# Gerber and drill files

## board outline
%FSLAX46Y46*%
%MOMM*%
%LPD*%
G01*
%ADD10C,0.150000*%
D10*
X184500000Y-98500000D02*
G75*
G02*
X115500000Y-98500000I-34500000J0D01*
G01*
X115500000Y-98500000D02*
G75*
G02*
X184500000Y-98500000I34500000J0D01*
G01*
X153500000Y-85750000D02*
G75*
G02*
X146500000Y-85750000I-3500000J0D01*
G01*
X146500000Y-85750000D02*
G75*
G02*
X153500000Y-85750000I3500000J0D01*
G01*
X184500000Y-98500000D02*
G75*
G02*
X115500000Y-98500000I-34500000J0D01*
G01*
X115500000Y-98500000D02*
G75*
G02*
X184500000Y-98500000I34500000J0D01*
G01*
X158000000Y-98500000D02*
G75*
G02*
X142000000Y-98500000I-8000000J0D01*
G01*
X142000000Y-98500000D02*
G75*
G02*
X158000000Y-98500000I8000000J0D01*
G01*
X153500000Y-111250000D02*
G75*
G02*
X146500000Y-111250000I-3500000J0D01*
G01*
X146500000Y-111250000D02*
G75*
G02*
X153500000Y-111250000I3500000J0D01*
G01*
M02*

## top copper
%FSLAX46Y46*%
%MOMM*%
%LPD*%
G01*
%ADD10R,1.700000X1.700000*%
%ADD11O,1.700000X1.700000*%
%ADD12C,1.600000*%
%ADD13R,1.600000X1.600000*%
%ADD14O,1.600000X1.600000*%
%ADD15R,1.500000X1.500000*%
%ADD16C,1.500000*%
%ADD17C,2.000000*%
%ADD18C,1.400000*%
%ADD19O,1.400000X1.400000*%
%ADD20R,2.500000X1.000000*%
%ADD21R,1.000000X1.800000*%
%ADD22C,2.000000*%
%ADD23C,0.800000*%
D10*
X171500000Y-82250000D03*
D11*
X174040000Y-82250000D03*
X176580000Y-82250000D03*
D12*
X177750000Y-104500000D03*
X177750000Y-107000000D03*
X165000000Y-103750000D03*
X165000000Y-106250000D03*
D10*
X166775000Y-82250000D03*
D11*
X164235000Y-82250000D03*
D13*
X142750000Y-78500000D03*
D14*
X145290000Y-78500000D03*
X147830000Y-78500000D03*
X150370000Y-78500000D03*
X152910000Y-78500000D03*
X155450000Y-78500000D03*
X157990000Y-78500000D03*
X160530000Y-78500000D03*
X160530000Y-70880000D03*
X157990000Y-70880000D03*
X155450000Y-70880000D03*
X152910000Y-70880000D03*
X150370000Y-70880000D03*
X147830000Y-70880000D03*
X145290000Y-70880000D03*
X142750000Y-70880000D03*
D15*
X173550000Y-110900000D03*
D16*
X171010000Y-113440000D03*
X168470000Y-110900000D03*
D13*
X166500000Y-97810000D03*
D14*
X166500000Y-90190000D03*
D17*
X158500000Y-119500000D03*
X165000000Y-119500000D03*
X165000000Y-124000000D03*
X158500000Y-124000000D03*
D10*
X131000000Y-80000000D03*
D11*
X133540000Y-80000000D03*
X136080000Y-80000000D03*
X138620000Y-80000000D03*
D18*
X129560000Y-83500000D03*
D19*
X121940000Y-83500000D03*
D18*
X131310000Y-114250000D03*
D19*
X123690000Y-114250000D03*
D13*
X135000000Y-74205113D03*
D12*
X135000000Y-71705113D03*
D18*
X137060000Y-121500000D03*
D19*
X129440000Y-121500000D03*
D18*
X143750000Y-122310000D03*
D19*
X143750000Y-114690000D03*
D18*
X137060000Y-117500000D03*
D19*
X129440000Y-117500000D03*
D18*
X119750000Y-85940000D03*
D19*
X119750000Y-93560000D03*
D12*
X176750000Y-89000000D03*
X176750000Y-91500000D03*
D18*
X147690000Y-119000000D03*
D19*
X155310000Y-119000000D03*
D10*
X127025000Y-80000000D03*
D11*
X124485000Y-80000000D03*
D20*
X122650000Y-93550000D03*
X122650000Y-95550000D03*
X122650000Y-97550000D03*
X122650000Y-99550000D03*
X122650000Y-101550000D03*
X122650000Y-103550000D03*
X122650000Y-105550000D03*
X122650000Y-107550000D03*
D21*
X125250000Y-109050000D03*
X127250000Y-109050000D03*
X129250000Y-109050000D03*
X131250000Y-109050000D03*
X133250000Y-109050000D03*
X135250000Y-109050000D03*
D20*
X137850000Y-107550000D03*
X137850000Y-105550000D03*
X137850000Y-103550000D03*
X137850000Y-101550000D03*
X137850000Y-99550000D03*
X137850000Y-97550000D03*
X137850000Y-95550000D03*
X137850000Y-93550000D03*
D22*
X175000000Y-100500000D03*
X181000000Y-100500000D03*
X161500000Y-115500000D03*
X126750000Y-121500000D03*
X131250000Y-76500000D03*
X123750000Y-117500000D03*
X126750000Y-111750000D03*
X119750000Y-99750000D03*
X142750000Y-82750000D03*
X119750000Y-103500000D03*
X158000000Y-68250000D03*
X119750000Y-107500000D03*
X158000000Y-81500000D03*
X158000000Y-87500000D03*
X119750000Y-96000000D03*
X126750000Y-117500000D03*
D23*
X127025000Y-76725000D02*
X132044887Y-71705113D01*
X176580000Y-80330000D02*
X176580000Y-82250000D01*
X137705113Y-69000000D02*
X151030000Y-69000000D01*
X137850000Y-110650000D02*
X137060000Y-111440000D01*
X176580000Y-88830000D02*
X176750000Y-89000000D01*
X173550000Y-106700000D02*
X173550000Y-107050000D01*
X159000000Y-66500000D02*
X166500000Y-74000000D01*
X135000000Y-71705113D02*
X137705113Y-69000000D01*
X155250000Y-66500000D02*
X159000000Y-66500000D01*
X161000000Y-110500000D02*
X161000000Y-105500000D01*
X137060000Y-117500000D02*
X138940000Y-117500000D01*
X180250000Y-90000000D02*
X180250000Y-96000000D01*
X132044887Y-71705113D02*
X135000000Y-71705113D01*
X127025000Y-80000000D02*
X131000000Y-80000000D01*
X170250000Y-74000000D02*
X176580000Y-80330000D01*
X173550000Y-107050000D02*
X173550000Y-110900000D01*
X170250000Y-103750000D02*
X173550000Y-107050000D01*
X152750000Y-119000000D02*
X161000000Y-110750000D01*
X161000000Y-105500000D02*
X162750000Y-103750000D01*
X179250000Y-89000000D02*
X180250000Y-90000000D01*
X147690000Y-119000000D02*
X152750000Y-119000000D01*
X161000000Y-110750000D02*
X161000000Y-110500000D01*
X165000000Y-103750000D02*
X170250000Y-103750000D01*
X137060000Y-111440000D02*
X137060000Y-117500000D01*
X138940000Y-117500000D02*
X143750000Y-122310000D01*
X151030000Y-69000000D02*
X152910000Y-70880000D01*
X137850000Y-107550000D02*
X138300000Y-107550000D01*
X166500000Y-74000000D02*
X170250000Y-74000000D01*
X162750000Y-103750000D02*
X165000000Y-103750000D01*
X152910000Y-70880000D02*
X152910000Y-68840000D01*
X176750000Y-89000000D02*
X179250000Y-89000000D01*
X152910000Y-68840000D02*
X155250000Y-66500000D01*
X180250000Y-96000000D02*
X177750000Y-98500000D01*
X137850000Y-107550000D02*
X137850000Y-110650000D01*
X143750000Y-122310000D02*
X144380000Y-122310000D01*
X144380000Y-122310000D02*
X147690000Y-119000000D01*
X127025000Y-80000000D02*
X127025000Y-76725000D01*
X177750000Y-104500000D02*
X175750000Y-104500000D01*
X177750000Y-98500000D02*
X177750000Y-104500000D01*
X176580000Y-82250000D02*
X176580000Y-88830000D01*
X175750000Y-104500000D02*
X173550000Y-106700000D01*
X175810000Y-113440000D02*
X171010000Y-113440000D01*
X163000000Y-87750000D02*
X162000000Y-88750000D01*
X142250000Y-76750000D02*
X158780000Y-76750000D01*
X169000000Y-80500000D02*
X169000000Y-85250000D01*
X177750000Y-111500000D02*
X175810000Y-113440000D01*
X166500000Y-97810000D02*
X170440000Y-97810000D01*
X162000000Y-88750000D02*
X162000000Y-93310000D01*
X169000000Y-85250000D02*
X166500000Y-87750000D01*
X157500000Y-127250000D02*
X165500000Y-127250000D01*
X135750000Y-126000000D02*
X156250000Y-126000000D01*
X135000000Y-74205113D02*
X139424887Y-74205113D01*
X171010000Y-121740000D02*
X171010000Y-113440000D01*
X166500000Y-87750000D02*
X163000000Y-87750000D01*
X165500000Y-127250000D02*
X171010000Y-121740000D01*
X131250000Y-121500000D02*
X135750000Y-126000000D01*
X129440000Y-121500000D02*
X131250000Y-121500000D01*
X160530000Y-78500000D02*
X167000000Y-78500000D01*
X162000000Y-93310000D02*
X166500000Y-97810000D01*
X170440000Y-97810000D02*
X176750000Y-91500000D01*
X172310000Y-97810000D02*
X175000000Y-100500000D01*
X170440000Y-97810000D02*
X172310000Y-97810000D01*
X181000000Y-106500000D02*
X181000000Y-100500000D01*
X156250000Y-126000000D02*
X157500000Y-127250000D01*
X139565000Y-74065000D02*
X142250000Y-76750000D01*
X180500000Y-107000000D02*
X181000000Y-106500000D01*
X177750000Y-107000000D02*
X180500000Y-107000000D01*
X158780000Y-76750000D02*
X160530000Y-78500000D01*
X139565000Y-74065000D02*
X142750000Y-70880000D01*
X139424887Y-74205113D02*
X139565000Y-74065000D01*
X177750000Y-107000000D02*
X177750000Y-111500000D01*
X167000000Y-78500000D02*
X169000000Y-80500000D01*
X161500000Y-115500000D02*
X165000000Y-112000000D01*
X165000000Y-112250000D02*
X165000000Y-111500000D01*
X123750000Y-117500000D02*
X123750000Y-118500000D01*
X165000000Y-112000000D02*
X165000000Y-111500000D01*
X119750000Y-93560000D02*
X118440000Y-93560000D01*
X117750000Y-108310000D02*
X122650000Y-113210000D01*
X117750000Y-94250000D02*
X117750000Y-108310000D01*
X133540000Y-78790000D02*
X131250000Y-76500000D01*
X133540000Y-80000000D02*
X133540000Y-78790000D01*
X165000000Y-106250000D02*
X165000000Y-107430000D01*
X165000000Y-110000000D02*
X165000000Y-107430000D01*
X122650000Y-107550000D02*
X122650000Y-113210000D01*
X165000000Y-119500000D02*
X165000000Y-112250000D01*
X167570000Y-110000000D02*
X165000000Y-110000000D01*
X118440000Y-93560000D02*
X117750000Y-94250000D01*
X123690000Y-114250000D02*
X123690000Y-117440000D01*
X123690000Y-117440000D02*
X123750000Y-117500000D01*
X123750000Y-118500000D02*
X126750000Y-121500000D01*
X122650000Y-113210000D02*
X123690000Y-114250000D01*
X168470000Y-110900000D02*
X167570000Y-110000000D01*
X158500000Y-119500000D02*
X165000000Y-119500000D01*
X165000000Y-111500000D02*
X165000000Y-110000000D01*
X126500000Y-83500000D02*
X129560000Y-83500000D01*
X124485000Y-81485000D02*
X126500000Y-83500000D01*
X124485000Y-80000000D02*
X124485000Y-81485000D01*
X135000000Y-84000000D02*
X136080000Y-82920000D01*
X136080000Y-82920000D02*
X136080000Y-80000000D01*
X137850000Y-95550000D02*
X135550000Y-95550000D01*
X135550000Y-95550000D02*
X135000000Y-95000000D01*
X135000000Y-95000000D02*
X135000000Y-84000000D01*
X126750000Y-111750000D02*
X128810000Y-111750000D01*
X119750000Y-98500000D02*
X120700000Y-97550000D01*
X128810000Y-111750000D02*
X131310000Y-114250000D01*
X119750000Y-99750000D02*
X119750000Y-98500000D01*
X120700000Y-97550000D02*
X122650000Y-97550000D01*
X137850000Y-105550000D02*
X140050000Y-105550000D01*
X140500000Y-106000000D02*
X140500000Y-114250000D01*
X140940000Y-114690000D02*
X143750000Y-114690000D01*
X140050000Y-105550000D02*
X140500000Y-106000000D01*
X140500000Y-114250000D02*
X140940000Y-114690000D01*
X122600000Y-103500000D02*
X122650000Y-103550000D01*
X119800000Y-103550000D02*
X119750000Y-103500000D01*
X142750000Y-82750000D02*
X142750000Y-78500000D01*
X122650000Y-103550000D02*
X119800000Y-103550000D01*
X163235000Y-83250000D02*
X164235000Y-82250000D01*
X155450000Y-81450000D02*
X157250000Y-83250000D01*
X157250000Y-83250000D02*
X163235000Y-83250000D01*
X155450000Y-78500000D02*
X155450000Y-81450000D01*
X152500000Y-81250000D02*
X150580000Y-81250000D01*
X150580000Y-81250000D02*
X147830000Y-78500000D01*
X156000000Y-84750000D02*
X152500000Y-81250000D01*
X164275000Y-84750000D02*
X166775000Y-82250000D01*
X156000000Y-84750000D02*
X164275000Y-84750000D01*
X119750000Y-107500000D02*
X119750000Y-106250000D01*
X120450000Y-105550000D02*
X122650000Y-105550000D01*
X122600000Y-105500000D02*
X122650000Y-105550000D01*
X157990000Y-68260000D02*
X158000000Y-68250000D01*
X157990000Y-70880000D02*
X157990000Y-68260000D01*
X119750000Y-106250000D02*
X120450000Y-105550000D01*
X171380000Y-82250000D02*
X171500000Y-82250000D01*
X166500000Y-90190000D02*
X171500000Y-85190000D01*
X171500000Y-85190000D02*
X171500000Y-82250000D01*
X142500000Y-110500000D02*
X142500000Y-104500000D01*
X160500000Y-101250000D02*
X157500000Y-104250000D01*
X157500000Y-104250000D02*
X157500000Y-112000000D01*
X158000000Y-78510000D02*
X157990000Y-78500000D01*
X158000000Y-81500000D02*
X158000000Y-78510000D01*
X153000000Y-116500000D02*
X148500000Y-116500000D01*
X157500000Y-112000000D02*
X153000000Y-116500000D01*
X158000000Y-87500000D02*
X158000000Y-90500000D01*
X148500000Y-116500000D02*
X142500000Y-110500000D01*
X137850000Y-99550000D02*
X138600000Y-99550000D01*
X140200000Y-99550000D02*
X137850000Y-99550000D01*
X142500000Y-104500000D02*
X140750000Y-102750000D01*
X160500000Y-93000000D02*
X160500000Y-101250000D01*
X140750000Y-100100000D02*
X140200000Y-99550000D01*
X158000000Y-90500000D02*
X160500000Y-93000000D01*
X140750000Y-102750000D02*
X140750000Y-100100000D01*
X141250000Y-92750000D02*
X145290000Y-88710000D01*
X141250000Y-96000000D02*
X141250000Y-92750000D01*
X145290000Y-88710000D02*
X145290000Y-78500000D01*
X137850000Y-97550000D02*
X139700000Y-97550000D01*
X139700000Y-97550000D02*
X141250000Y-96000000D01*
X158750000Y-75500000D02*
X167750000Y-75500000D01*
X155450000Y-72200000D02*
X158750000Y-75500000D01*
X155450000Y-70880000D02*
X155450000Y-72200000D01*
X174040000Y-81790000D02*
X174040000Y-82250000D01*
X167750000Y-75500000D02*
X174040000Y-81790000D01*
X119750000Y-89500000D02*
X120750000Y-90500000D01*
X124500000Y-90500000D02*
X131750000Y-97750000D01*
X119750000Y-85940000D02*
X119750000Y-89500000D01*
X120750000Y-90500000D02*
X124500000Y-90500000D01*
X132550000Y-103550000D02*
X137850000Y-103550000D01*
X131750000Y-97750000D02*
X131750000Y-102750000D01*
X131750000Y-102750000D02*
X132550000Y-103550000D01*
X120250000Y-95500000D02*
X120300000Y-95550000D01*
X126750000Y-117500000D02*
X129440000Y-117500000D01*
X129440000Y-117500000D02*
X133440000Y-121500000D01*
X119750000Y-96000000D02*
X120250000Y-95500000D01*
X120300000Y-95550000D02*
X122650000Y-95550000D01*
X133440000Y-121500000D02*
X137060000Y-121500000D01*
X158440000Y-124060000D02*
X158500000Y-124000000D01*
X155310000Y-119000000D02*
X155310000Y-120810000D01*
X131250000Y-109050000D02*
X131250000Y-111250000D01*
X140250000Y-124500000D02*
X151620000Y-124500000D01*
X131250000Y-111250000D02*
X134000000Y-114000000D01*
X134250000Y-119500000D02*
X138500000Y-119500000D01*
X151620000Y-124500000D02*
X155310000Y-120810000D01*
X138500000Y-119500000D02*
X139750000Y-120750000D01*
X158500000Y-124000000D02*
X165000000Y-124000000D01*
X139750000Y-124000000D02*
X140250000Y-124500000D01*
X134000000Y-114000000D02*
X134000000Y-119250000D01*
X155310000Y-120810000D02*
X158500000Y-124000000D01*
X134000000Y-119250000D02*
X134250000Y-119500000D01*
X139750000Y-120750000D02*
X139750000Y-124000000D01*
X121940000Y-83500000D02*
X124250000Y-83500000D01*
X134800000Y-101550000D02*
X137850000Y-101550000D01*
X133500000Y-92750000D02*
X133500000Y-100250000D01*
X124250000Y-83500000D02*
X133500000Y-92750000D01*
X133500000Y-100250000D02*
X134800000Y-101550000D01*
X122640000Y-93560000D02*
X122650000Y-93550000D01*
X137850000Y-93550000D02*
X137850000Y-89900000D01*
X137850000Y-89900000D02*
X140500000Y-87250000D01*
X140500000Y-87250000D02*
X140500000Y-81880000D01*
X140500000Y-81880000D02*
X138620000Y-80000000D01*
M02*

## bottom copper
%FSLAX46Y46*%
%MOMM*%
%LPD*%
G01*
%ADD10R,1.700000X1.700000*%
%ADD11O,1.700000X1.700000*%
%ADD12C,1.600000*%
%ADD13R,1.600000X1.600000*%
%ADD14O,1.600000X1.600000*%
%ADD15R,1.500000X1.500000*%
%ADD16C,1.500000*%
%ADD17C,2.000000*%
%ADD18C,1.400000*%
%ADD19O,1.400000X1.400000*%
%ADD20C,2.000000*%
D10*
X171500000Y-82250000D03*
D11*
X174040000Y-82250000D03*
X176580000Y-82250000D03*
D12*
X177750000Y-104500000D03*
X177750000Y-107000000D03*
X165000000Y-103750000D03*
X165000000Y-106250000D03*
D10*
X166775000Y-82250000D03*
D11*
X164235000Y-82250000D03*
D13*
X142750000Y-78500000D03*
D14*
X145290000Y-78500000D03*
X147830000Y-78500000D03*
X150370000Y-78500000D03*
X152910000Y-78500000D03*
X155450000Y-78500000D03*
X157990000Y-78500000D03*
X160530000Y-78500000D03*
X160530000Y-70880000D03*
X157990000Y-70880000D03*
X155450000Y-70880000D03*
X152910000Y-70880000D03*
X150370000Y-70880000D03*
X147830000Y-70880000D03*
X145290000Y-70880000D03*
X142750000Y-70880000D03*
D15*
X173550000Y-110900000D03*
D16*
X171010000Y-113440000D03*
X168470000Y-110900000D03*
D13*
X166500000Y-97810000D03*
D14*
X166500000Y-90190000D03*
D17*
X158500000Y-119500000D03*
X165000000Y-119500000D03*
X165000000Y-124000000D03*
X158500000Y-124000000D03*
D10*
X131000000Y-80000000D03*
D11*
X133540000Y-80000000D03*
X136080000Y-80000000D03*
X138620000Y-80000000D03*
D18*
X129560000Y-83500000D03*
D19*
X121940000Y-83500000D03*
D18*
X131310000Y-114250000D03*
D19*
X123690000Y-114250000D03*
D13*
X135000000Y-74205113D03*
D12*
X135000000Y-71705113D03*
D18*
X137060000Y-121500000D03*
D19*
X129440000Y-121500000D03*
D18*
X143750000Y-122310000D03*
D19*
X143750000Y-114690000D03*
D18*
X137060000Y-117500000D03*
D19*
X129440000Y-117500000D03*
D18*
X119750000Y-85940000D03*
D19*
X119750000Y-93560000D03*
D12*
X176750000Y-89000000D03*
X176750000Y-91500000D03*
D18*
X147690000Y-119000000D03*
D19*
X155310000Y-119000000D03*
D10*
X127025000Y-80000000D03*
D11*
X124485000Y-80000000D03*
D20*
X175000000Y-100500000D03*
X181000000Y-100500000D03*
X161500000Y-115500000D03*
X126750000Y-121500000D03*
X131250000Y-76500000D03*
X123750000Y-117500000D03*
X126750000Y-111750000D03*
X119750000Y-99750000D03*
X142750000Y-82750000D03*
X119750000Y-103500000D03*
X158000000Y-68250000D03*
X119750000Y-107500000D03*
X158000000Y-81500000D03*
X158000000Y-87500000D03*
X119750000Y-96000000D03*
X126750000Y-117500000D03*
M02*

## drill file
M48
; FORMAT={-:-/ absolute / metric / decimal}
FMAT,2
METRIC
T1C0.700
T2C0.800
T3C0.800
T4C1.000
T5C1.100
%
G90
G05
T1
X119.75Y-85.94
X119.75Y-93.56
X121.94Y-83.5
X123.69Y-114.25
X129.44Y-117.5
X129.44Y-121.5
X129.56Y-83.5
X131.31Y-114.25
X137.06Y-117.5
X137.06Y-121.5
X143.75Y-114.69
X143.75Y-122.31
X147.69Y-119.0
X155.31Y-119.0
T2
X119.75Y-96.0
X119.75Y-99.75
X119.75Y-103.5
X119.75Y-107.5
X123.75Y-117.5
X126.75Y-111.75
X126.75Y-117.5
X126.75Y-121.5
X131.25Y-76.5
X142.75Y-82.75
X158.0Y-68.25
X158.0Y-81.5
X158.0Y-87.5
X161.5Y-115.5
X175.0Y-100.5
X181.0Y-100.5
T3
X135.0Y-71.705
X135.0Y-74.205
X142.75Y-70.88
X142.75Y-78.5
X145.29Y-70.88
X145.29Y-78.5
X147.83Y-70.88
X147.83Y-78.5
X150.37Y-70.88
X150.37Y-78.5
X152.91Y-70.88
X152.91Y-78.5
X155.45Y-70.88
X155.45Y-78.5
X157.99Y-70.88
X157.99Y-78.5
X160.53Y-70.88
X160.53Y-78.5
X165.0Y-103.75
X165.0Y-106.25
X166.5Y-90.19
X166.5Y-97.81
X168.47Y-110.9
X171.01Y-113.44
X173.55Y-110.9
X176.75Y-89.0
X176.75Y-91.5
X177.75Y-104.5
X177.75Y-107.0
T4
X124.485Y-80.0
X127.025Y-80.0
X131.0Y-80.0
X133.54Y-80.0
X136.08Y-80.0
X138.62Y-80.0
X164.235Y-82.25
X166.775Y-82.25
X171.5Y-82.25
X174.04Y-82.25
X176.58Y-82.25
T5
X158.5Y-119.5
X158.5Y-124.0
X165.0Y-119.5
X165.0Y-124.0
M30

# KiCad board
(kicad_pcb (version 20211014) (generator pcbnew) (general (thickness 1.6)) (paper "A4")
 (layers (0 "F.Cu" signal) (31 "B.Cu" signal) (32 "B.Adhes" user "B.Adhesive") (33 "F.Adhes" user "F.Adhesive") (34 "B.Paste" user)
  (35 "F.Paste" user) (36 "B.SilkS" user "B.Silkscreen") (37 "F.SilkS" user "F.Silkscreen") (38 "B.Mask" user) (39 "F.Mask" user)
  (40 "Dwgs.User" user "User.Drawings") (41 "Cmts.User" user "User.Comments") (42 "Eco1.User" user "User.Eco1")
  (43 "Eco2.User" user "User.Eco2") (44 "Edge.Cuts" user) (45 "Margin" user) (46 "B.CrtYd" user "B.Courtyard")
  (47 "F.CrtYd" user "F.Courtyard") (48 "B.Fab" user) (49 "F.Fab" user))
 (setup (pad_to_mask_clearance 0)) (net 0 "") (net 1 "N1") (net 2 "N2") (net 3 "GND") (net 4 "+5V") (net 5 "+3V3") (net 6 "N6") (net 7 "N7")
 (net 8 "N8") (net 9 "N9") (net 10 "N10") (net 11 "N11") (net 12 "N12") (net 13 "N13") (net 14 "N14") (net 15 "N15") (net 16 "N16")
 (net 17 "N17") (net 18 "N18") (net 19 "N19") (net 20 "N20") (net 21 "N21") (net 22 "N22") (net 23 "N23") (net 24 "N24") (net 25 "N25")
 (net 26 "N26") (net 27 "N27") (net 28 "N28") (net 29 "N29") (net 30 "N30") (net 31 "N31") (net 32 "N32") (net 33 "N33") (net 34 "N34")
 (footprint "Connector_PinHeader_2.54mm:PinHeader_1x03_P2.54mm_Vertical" (layer "F.Cu") (at 171.5 82.25 90)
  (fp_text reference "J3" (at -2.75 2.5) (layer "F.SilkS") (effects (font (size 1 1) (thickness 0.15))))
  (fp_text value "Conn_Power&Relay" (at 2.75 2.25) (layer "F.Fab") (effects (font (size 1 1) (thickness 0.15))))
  (pad "1" thru_hole rect locked (at 0 0 90) (size 1.7 1.7) (drill 1) (layers *.Cu *.Mask) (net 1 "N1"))
  (pad "2" thru_hole oval locked (at 0 2.54 90) (size 1.7 1.7) (drill 1) (layers *.Cu *.Mask) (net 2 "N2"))
  (pad "3" thru_hole oval locked (at 0 5.08 90) (size 1.7 1.7) (drill 1) (layers *.Cu *.Mask) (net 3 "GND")))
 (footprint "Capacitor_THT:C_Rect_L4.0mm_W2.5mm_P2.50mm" (layer "F.Cu") (at 177.75 104.5 -90)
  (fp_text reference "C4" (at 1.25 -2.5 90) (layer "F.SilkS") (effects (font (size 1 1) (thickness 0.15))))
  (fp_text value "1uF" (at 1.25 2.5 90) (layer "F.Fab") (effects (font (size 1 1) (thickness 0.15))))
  (pad "1" thru_hole circle locked (at 0 0 270) (size 1.6 1.6) (drill 0.8) (layers *.Cu *.Mask) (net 3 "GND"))
  (pad "2" thru_hole circle locked (at 2.5 0 270) (size 1.6 1.6) (drill 0.8) (layers *.Cu *.Mask) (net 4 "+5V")))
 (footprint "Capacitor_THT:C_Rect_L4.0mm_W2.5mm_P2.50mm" (layer "F.Cu") (at 165 103.75 -90)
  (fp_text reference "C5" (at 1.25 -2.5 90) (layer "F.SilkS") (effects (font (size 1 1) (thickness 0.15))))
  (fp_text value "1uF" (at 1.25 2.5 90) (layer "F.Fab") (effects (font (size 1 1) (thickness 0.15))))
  (pad "1" thru_hole circle locked (at 0 0 270) (size 1.6 1.6) (drill 0.8) (layers *.Cu *.Mask) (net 3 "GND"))
  (pad "2" thru_hole circle locked (at 2.5 0 270) (size 1.6 1.6) (drill 0.8) (layers *.Cu *.Mask) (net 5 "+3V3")))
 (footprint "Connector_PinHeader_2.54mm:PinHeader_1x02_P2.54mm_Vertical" (layer "F.Cu") (at 166.775 82.25 -90)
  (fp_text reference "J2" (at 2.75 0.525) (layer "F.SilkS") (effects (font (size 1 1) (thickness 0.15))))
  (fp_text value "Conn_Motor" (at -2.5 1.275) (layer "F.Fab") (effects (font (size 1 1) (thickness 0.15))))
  (pad "1" thru_hole rect locked (at 0 0 270) (size 1.7 1.7) (drill 1) (layers *.Cu *.Mask) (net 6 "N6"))
  (pad "2" thru_hole oval locked (at 0 2.54 270) (size 1.7 1.7) (drill 1) (layers *.Cu *.Mask) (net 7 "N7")))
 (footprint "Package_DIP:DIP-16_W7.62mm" (layer "F.Cu") (at 142.75 78.5 90)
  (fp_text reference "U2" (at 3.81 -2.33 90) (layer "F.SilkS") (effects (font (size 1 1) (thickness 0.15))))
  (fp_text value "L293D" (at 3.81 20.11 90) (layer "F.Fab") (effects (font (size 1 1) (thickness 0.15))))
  (pad "1" thru_hole rect locked (at 0 0 90) (size 1.6 1.6) (drill 0.8) (layers *.Cu *.Mask) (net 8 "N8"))
  (pad "2" thru_hole oval locked (at 0 2.54 90) (size 1.6 1.6) (drill 0.8) (layers *.Cu *.Mask) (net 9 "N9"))
  (pad "3" thru_hole oval locked (at 0 5.08 90) (size 1.6 1.6) (drill 0.8) (layers *.Cu *.Mask) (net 6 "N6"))
  (pad "4" thru_hole oval locked (at 0 7.62 90) (size 1.6 1.6) (drill 0.8) (layers *.Cu *.Mask) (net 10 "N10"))
  (pad "5" thru_hole oval locked (at 0 10.16 90) (size 1.6 1.6) (drill 0.8) (layers *.Cu *.Mask) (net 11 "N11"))
  (pad "6" thru_hole oval locked (at 0 12.7 90) (size 1.6 1.6) (drill 0.8) (layers *.Cu *.Mask) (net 7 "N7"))
  (pad "7" thru_hole oval locked (at 0 15.24 90) (size 1.6 1.6) (drill 0.8) (layers *.Cu *.Mask) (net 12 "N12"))
  (pad "8" thru_hole oval locked (at 0 17.78 90) (size 1.6 1.6) (drill 0.8) (layers *.Cu *.Mask) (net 4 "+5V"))
  (pad "9" thru_hole oval locked (at 7.62 17.78 90) (size 1.6 1.6) (drill 0.8) (layers *.Cu *.Mask) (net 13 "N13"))
  (pad "10" thru_hole oval locked (at 7.62 15.24 90) (size 1.6 1.6) (drill 0.8) (layers *.Cu *.Mask) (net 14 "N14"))
  (pad "11" thru_hole oval locked (at 7.62 12.7 90) (size 1.6 1.6) (drill 0.8) (layers *.Cu *.Mask) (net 2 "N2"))
  (pad "12" thru_hole oval locked (at 7.62 10.16 90) (size 1.6 1.6) (drill 0.8) (layers *.Cu *.Mask) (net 3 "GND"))
  (pad "13" thru_hole oval locked (at 7.62 7.62 90) (size 1.6 1.6) (drill 0.8) (layers *.Cu *.Mask) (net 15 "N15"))
  (pad "14" thru_hole oval locked (at 7.62 5.08 90) (size 1.6 1.6) (drill 0.8) (layers *.Cu *.Mask) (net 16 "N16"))
  (pad "15" thru_hole oval locked (at 7.62 2.54 90) (size 1.6 1.6) (drill 0.8) (layers *.Cu *.Mask) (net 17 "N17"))
  (pad "16" thru_hole oval locked (at 7.62 0 90) (size 1.6 1.6) (drill 0.8) (layers *.Cu *.Mask) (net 4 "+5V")))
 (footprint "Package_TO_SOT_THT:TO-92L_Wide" (layer "F.Cu") (at 173.55 110.9 180)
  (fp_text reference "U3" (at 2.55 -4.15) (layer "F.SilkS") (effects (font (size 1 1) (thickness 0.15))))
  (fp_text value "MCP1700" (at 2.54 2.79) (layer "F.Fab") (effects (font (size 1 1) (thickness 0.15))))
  (pad "1" thru_hole rect locked (at 0 0 180) (size 1.5 1.5) (drill 0.8) (layers *.Cu *.Mask) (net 3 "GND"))
  (pad "2" thru_hole circle locked (at 2.54 -2.54 180) (size 1.5 1.5) (drill 0.8) (layers *.Cu *.Mask) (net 4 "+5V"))
  (pad "3" thru_hole circle locked (at 5.08 0 180) (size 1.5 1.5) (drill 0.8) (layers *.Cu *.Mask) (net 5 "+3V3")))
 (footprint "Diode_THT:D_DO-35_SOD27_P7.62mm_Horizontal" (layer "F.Cu") (at 166.5 97.81 90)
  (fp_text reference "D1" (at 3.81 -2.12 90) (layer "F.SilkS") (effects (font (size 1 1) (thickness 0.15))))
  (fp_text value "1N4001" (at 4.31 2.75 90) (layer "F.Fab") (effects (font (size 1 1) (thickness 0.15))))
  (pad "1" thru_hole rect locked (at 0 0 90) (size 1.6 1.6) (drill 0.8) (layers *.Cu *.Mask) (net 4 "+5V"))
  (pad "2" thru_hole oval locked (at 7.62 0 90) (size 1.6 1.6) (drill 0.8) (layers *.Cu *.Mask) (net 1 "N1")))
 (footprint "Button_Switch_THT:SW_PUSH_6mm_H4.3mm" (layer "F.Cu") (at 158.5 119.5)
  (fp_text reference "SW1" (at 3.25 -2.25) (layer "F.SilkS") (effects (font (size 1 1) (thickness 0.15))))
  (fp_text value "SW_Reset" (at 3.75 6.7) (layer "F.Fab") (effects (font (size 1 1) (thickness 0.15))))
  (pad "1" thru_hole circle locked (at 0 0 90) (size 2 2) (drill 1.1) (layers *.Cu *.Mask) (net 5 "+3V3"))
  (pad "1" thru_hole circle locked (at 6.5 0 90) (size 2 2) (drill 1.1) (layers *.Cu *.Mask) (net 5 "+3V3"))
  (pad "2" thru_hole circle locked (at 6.5 4.5 90) (size 2 2) (drill 1.1) (layers *.Cu *.Mask) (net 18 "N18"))
  (pad "2" thru_hole circle locked (at 0 4.5 90) (size 2 2) (drill 1.1) (layers *.Cu *.Mask) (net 18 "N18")))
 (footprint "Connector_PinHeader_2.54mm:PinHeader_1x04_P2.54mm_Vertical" (layer "F.Cu") (at 131 80 90)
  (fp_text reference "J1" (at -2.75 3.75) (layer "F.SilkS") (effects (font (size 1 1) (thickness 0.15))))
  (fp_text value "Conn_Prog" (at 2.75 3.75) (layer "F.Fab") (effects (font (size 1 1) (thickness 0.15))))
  (pad "1" thru_hole rect locked (at 0 0 90) (size 1.7 1.7) (drill 1) (layers *.Cu *.Mask) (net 3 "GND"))
  (pad "2" thru_hole oval locked (at 0 2.54 90) (size 1.7 1.7) (drill 1) (layers *.Cu *.Mask) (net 5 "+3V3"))
  (pad "3" thru_hole oval locked (at 0 5.08 90) (size 1.7 1.7) (drill 1) (layers *.Cu *.Mask) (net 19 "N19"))
  (pad "4" thru_hole oval locked (at 0 7.62 90) (size 1.7 1.7) (drill 1) (layers *.Cu *.Mask) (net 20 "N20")))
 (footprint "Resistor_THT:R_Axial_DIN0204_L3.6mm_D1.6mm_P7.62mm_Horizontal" (layer "F.Cu") (at 129.56 83.5 180)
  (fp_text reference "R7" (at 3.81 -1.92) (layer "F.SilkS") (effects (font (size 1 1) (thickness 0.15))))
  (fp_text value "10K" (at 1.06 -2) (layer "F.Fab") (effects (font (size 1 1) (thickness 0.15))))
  (pad "1" thru_hole circle locked (at 0 0 180) (size 1.4 1.4) (drill 0.7) (layers *.Cu *.Mask) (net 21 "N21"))
  (pad "2" thru_hole oval locked (at 7.62 0 180) (size 1.4 1.4) (drill 0.7) (layers *.Cu *.Mask) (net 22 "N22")))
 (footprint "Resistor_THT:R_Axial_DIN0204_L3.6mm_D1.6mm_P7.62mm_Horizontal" (layer "F.Cu") (at 131.31 114.25 180)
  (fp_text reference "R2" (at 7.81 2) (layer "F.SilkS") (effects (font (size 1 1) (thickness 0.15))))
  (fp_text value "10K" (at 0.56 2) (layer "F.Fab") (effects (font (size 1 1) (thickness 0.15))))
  (pad "1" thru_hole circle locked (at 0 0 180) (size 1.4 1.4) (drill 0.7) (layers *.Cu *.Mask) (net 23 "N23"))
  (pad "2" thru_hole oval locked (at 7.62 0 180) (size 1.4 1.4) (drill 0.7) (layers *.Cu *.Mask) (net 5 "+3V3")))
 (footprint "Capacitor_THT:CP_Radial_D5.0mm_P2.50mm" (layer "F.Cu") (at 135 74.205113 90)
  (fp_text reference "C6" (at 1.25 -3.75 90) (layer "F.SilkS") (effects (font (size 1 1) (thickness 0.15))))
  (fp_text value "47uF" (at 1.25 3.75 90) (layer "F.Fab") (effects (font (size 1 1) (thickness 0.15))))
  (pad "1" thru_hole rect locked (at 0 0 90) (size 1.6 1.6) (drill 0.8) (layers *.Cu *.Mask) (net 4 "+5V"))
  (pad "2" thru_hole circle locked (at 2.5 0 90) (size 1.6 1.6) (drill 0.8) (layers *.Cu *.Mask) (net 3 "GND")))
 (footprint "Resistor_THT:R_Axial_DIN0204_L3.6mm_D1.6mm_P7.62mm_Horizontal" (layer "F.Cu") (at 137.06 121.5 180)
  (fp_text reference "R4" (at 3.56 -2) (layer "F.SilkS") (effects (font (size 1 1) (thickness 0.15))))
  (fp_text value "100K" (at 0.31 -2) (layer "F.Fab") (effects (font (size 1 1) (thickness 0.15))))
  (pad "1" thru_hole circle locked (at 0 0 180) (size 1.4 1.4) (drill 0.7) (layers *.Cu *.Mask) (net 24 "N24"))
  (pad "2" thru_hole oval locked (at 7.62 0 180) (size 1.4 1.4) (drill 0.7) (layers *.Cu *.Mask) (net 4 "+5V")))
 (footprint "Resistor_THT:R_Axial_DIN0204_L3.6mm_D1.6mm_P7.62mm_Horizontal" (layer "F.Cu") (at 143.75 122.31 90)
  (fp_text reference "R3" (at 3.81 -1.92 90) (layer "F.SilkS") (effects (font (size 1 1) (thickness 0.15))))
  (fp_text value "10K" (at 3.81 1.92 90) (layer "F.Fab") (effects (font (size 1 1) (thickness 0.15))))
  (pad "1" thru_hole circle locked (at 0 0 90) (size 1.4 1.4) (drill 0.7) (layers *.Cu *.Mask) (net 3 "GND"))
  (pad "2" thru_hole oval locked (at 7.62 0 90) (size 1.4 1.4) (drill 0.7) (layers *.Cu *.Mask) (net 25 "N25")))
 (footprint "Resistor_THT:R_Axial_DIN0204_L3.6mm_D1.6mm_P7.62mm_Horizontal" (layer "F.Cu") (at 137.06 117.5 180)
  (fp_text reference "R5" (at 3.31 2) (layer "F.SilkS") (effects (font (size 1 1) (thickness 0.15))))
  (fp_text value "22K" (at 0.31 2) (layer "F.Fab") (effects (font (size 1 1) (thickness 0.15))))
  (pad "1" thru_hole circle locked (at 0 0 180) (size 1.4 1.4) (drill 0.7) (layers *.Cu *.Mask) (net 3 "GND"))
  (pad "2" thru_hole oval locked (at 7.62 0 180) (size 1.4 1.4) (drill 0.7) (layers *.Cu *.Mask) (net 24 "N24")))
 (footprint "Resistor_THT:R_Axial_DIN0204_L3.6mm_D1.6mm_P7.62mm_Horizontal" (layer "F.Cu") (at 119.75 85.94 -90)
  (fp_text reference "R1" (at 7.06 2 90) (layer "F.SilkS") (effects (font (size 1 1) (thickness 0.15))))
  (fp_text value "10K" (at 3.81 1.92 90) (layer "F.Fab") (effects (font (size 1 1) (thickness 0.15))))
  (pad "1" thru_hole circle locked (at 0 0 270) (size 1.4 1.4) (drill 0.7) (layers *.Cu *.Mask) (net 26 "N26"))
  (pad "2" thru_hole oval locked (at 7.62 0 270) (size 1.4 1.4) (drill 0.7) (layers *.Cu *.Mask) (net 5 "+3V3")))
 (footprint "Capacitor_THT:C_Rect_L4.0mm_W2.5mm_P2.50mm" (layer "F.Cu") (at 176.75 89 -90)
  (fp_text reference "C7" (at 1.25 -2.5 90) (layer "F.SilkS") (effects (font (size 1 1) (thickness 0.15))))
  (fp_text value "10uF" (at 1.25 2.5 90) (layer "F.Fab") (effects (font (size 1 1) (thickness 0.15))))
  (pad "1" thru_hole circle locked (at 0 0 270) (size 1.6 1.6) (drill 0.8) (layers *.Cu *.Mask) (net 3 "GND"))
  (pad "2" thru_hole circle locked (at 2.5 0 270) (size 1.6 1.6) (drill 0.8) (layers *.Cu *.Mask) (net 4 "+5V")))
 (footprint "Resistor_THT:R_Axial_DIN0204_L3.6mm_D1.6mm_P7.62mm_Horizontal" (layer "F.Cu") (at 147.69 119)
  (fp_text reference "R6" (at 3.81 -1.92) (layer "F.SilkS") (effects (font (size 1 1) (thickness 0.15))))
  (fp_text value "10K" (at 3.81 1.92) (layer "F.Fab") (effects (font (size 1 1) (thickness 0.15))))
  (pad "1" thru_hole circle locked (at 0 0) (size 1.4 1.4) (drill 0.7) (layers *.Cu *.Mask) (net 3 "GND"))
  (pad "2" thru_hole oval locked (at 7.62 0) (size 1.4 1.4) (drill 0.7) (layers *.Cu *.Mask) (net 18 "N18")))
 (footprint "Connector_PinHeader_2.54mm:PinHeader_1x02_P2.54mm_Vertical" (layer "F.Cu") (at 127.025 80 -90)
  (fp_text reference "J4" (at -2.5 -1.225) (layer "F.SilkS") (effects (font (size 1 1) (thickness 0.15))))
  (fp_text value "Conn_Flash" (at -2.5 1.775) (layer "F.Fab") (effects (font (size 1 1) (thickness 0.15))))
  (pad "1" thru_hole rect locked (at 0 0 270) (size 1.7 1.7) (drill 1) (layers *.Cu *.Mask) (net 3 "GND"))
  (pad "2" thru_hole oval locked (at 0 2.54 270) (size 1.7 1.7) (drill 1) (layers *.Cu *.Mask) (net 21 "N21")))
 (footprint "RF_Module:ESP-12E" (layer "F.Cu") (at 130.25 97.05)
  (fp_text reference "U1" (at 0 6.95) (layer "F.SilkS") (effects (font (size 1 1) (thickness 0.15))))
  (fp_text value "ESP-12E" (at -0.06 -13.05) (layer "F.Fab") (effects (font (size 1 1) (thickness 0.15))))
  (pad "1" smd rect locked (at -7.6 -3.5) (size 2.5 1) (layers "F.Cu" "F.Paste" "F.Mask") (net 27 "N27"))
  (pad "2" smd rect locked (at -7.6 -1.5) (size 2.5 1) (layers "F.Cu" "F.Paste" "F.Mask") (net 24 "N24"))
  (pad "3" smd rect locked (at -7.6 0.5) (size 2.5 1) (layers "F.Cu" "F.Paste" "F.Mask") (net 23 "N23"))
  (pad "4" smd rect locked (at -7.6 2.5) (size 2.5 1) (layers "F.Cu" "F.Paste" "F.Mask") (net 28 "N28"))
  (pad "5" smd rect locked (at -7.6 4.5) (size 2.5 1) (layers "F.Cu" "F.Paste" "F.Mask") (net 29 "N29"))
  (pad "6" smd rect locked (at -7.6 6.5) (size 2.5 1) (layers "F.Cu" "F.Paste" "F.Mask") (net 8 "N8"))
  (pad "7" smd rect locked (at -7.6 8.5) (size 2.5 1) (layers "F.Cu" "F.Paste" "F.Mask") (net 14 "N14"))
  (pad "8" smd rect locked (at -7.6 10.5) (size 2.5 1) (layers "F.Cu" "F.Paste" "F.Mask") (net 5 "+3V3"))
  (pad "9" smd rect locked (at -5 12) (size 1 1.8) (layers "F.Cu" "F.Paste" "F.Mask") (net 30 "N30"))
  (pad "10" smd rect locked (at -3 12) (size 1 1.8) (layers "F.Cu" "F.Paste" "F.Mask") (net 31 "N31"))
  (pad "11" smd rect locked (at -1 12) (size 1 1.8) (layers "F.Cu" "F.Paste" "F.Mask") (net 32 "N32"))
  (pad "12" smd rect locked (at 1 12) (size 1 1.8) (layers "F.Cu" "F.Paste" "F.Mask") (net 18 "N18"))
  (pad "13" smd rect locked (at 3 12) (size 1 1.8) (layers "F.Cu" "F.Paste" "F.Mask") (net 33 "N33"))
  (pad "14" smd rect locked (at 5 12) (size 1 1.8) (layers "F.Cu" "F.Paste" "F.Mask") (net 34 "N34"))
  (pad "15" smd rect locked (at 7.6 10.5) (size 2.5 1) (layers "F.Cu" "F.Paste" "F.Mask") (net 3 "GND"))
  (pad "16" smd rect locked (at 7.6 8.5) (size 2.5 1) (layers "F.Cu" "F.Paste" "F.Mask") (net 25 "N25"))
  (pad "17" smd rect locked (at 7.6 6.5) (size 2.5 1) (layers "F.Cu" "F.Paste" "F.Mask") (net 26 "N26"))
  (pad "18" smd rect locked (at 7.6 4.5) (size 2.5 1) (layers "F.Cu" "F.Paste" "F.Mask") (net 22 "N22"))
  (pad "19" smd rect locked (at 7.6 2.5) (size 2.5 1) (layers "F.Cu" "F.Paste" "F.Mask") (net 12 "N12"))
  (pad "20" smd rect locked (at 7.6 0.5) (size 2.5 1) (layers "F.Cu" "F.Paste" "F.Mask") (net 9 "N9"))
  (pad "21" smd rect locked (at 7.6 -1.5) (size 2.5 1) (layers "F.Cu" "F.Paste" "F.Mask") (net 19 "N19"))
  (pad "22" smd rect locked (at 7.6 -3.5) (size 2.5 1) (layers "F.Cu" "F.Paste" "F.Mask") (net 20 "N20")))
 (gr_circle (center 150 98.5) (end 184.5 98.5) (layer "Edge.Cuts") (width 0.15) (fill none))
 (gr_circle (center 150 85.75) (end 153.5 85.75) (layer "Edge.Cuts") (width 0.15) (fill none))
 (gr_circle (center 150 98.5) (end 184.5 98.5) (layer "Edge.Cuts") (width 0.15) (fill none))
 (gr_circle (center 150 98.5) (end 158 98.5) (layer "Edge.Cuts") (width 0.15) (fill none))
 (gr_circle (center 150 111.25) (end 153.5 111.25) (layer "Edge.Cuts") (width 0.15) (fill none))
 (segment (start 127.025 76.725) (end 132.044887 71.705113) (width 0.8) (layer "F.Cu") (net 3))
 (segment (start 176.58 80.33) (end 176.58 82.25) (width 0.8) (layer "F.Cu") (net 3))
 (segment (start 137.705113 69) (end 151.03 69) (width 0.8) (layer "F.Cu") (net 3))
 (segment (start 137.85 110.65) (end 137.06 111.44) (width 0.8) (layer "F.Cu") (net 3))
 (segment (start 176.58 88.83) (end 176.75 89) (width 0.8) (layer "F.Cu") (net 3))
 (segment (start 173.55 106.7) (end 173.55 107.05) (width 0.8) (layer "F.Cu") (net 3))
 (segment (start 159 66.5) (end 166.5 74) (width 0.8) (layer "F.Cu") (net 3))
 (segment (start 135 71.705113) (end 137.705113 69) (width 0.8) (layer "F.Cu") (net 3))
 (segment (start 155.25 66.5) (end 159 66.5) (width 0.8) (layer "F.Cu") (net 3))
 (segment (start 161 110.5) (end 161 105.5) (width 0.8) (layer "F.Cu") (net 3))
 (segment (start 137.06 117.5) (end 138.94 117.5) (width 0.8) (layer "F.Cu") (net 3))
 (segment (start 180.25 90) (end 180.25 96) (width 0.8) (layer "F.Cu") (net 3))
 (segment (start 132.044887 71.705113) (end 135 71.705113) (width 0.8) (layer "F.Cu") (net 3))
 (segment (start 127.025 80) (end 131 80) (width 0.8) (layer "F.Cu") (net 3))
 (segment (start 170.25 74) (end 176.58 80.33) (width 0.8) (layer "F.Cu") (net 3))
 (segment (start 173.55 107.05) (end 173.55 110.9) (width 0.8) (layer "F.Cu") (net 3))
 (segment (start 170.25 103.75) (end 173.55 107.05) (width 0.8) (layer "F.Cu") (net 3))
 (segment (start 152.75 119) (end 161 110.75) (width 0.8) (layer "F.Cu") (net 3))
 (segment (start 161 105.5) (end 162.75 103.75) (width 0.8) (layer "F.Cu") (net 3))
 (segment (start 179.25 89) (end 180.25 90) (width 0.8) (layer "F.Cu") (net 3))
 (segment (start 147.69 119) (end 152.75 119) (width 0.8) (layer "F.Cu") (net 3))
 (segment (start 161 110.75) (end 161 110.5) (width 0.8) (layer "F.Cu") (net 3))
 (segment (start 165 103.75) (end 170.25 103.75) (width 0.8) (layer "F.Cu") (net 3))
 (segment (start 137.06 111.44) (end 137.06 117.5) (width 0.8) (layer "F.Cu") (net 3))
 (segment (start 138.94 117.5) (end 143.75 122.31) (width 0.8) (layer "F.Cu") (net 3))
 (segment (start 151.03 69) (end 152.91 70.88) (width 0.8) (layer "F.Cu") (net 3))
 (segment (start 137.85 107.55) (end 138.3 107.55) (width 0.8) (layer "F.Cu") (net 3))
 (segment (start 166.5 74) (end 170.25 74) (width 0.8) (layer "F.Cu") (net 3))
 (segment (start 162.75 103.75) (end 165 103.75) (width 0.8) (layer "F.Cu") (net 3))
 (segment (start 152.91 70.88) (end 152.91 68.84) (width 0.8) (layer "F.Cu") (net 3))
 (segment (start 176.75 89) (end 179.25 89) (width 0.8) (layer "F.Cu") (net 3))
 (segment (start 152.91 68.84) (end 155.25 66.5) (width 0.8) (layer "F.Cu") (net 3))
 (segment (start 180.25 96) (end 177.75 98.5) (width 0.8) (layer "F.Cu") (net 3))
 (segment (start 137.85 107.55) (end 137.85 110.65) (width 0.8) (layer "F.Cu") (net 3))
 (segment (start 143.75 122.31) (end 144.38 122.31) (width 0.8) (layer "F.Cu") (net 3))
 (segment (start 144.38 122.31) (end 147.69 119) (width 0.8) (layer "F.Cu") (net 3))
 (segment (start 127.025 80) (end 127.025 76.725) (width 0.8) (layer "F.Cu") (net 3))
 (segment (start 177.75 104.5) (end 175.75 104.5) (width 0.8) (layer "F.Cu") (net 3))
 (segment (start 177.75 98.5) (end 177.75 104.5) (width 0.8) (layer "F.Cu") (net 3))
 (segment (start 176.58 82.25) (end 176.58 88.83) (width 0.8) (layer "F.Cu") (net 3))
 (segment (start 175.75 104.5) (end 173.55 106.7) (width 0.8) (layer "F.Cu") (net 3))
 (segment (start 175.81 113.44) (end 171.01 113.44) (width 0.8) (layer "F.Cu") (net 4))
 (segment (start 163 87.75) (end 162 88.75) (width 0.8) (layer "F.Cu") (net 4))
 (segment (start 142.25 76.75) (end 158.78 76.75) (width 0.8) (layer "F.Cu") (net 4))
 (segment (start 169 80.5) (end 169 85.25) (width 0.8) (layer "F.Cu") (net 4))
 (segment (start 177.75 111.5) (end 175.81 113.44) (width 0.8) (layer "F.Cu") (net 4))
 (segment (start 166.5 97.81) (end 170.44 97.81) (width 0.8) (layer "F.Cu") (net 4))
 (segment (start 162 88.75) (end 162 93.31) (width 0.8) (layer "F.Cu") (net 4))
 (segment (start 169 85.25) (end 166.5 87.75) (width 0.8) (layer "F.Cu") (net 4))
 (segment (start 157.5 127.25) (end 165.5 127.25) (width 0.8) (layer "F.Cu") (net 4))
 (segment (start 135.75 126) (end 156.25 126) (width 0.8) (layer "F.Cu") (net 4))
 (segment (start 135 74.205113) (end 139.424887 74.205113) (width 0.8) (layer "F.Cu") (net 4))
 (segment (start 171.01 121.74) (end 171.01 113.44) (width 0.8) (layer "F.Cu") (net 4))
 (segment (start 166.5 87.75) (end 163 87.75) (width 0.8) (layer "F.Cu") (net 4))
 (segment (start 165.5 127.25) (end 171.01 121.74) (width 0.8) (layer "F.Cu") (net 4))
 (segment (start 131.25 121.5) (end 135.75 126) (width 0.8) (layer "F.Cu") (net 4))
 (segment (start 129.44 121.5) (end 131.25 121.5) (width 0.8) (layer "F.Cu") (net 4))
 (segment (start 160.53 78.5) (end 167 78.5) (width 0.8) (layer "F.Cu") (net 4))
 (segment (start 162 93.31) (end 166.5 97.81) (width 0.8) (layer "F.Cu") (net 4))
 (segment (start 170.44 97.81) (end 176.75 91.5) (width 0.8) (layer "F.Cu") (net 4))
 (segment (start 172.31 97.81) (end 175 100.5) (width 0.8) (layer "F.Cu") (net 4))
 (segment (start 170.44 97.81) (end 172.31 97.81) (width 0.8) (layer "F.Cu") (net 4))
 (segment (start 181 106.5) (end 181 100.5) (width 0.8) (layer "F.Cu") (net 4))
 (segment (start 156.25 126) (end 157.5 127.25) (width 0.8) (layer "F.Cu") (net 4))
 (segment (start 139.565 74.065) (end 142.25 76.75) (width 0.8) (layer "F.Cu") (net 4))
 (segment (start 180.5 107) (end 181 106.5) (width 0.8) (layer "F.Cu") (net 4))
 (segment (start 177.75 107) (end 180.5 107) (width 0.8) (layer "F.Cu") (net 4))
 (segment (start 158.78 76.75) (end 160.53 78.5) (width 0.8) (layer "F.Cu") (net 4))
 (segment (start 139.565 74.065) (end 142.75 70.88) (width 0.8) (layer "F.Cu") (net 4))
 (segment (start 139.424887 74.205113) (end 139.565 74.065) (width 0.8) (layer "F.Cu") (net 4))
 (segment (start 177.75 107) (end 177.75 111.5) (width 0.8) (layer "F.Cu") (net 4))
 (segment (start 167 78.5) (end 169 80.5) (width 0.8) (layer "F.Cu") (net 4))
 (via (at 175 100.5) (size 2) (drill 0.8) (layers "F.Cu" "B.Cu") (free) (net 4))
 (via (at 181 100.5) (size 2) (drill 0.8) (layers "F.Cu" "B.Cu") (free) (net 4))
 (segment (start 161.5 115.5) (end 165 112) (width 0.8) (layer "F.Cu") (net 5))
 (segment (start 165 112.25) (end 165 111.5) (width 0.8) (layer "F.Cu") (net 5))
 (segment (start 123.75 117.5) (end 123.75 118.5) (width 0.8) (layer "F.Cu") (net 5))
 (segment (start 165 112) (end 165 111.5) (width 0.8) (layer "F.Cu") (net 5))
 (segment (start 119.75 93.56) (end 118.44 93.56) (width 0.8) (layer "F.Cu") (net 5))
 (segment (start 117.75 108.31) (end 122.65 113.21) (width 0.8) (layer "F.Cu") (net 5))
 (segment (start 117.75 94.25) (end 117.75 108.31) (width 0.8) (layer "F.Cu") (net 5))
 (segment (start 133.54 78.79) (end 131.25 76.5) (width 0.8) (layer "F.Cu") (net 5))
 (segment (start 133.54 80) (end 133.54 78.79) (width 0.8) (layer "F.Cu") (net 5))
 (segment (start 165 106.25) (end 165 107.43) (width 0.8) (layer "F.Cu") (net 5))
 (segment (start 165 110) (end 165 107.43) (width 0.8) (layer "F.Cu") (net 5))
 (segment (start 122.65 107.55) (end 122.65 113.21) (width 0.8) (layer "F.Cu") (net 5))
 (segment (start 165 119.5) (end 165 112.25) (width 0.8) (layer "F.Cu") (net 5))
 (segment (start 167.57 110) (end 165 110) (width 0.8) (layer "F.Cu") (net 5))
 (segment (start 118.44 93.56) (end 117.75 94.25) (width 0.8) (layer "F.Cu") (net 5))
 (segment (start 123.69 114.25) (end 123.69 117.44) (width 0.8) (layer "F.Cu") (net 5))
 (segment (start 123.69 117.44) (end 123.75 117.5) (width 0.8) (layer "F.Cu") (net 5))
 (segment (start 123.75 118.5) (end 126.75 121.5) (width 0.8) (layer "F.Cu") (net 5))
 (segment (start 122.65 113.21) (end 123.69 114.25) (width 0.8) (layer "F.Cu") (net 5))
 (segment (start 168.47 110.9) (end 167.57 110) (width 0.8) (layer "F.Cu") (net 5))
 (segment (start 158.5 119.5) (end 165 119.5) (width 0.8) (layer "F.Cu") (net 5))
 (segment (start 165 111.5) (end 165 110) (width 0.8) (layer "F.Cu") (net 5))
 (via (at 161.5 115.5) (size 2) (drill 0.8) (layers "F.Cu" "B.Cu") (free) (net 5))
 (via (at 126.75 121.5) (size 2) (drill 0.8) (layers "F.Cu" "B.Cu") (free) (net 5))
 (via (at 131.25 76.5) (size 2) (drill 0.8) (layers "F.Cu" "B.Cu") (free) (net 5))
 (via (at 123.75 117.5) (size 2) (drill 0.8) (layers "F.Cu" "B.Cu") (free) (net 5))
 (segment (start 126.5 83.5) (end 129.56 83.5) (width 0.8) (layer "F.Cu") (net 21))
 (segment (start 124.485 81.485) (end 126.5 83.5) (width 0.8) (layer "F.Cu") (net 21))
 (segment (start 124.485 80) (end 124.485 81.485) (width 0.8) (layer "F.Cu") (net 21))
 (segment (start 135 84) (end 136.08 82.92) (width 0.8) (layer "F.Cu") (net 19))
 (segment (start 136.08 82.92) (end 136.08 80) (width 0.8) (layer "F.Cu") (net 19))
 (segment (start 137.85 95.55) (end 135.55 95.55) (width 0.8) (layer "F.Cu") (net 19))
 (segment (start 135.55 95.55) (end 135 95) (width 0.8) (layer "F.Cu") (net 19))
 (segment (start 135 95) (end 135 84) (width 0.8) (layer "F.Cu") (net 19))
 (segment (start 126.75 111.75) (end 128.81 111.75) (width 0.8) (layer "F.Cu") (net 23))
 (segment (start 119.75 98.5) (end 120.7 97.55) (width 0.8) (layer "F.Cu") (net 23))
 (segment (start 128.81 111.75) (end 131.31 114.25) (width 0.8) (layer "F.Cu") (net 23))
 (segment (start 119.75 99.75) (end 119.75 98.5) (width 0.8) (layer "F.Cu") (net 23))
 (segment (start 120.7 97.55) (end 122.65 97.55) (width 0.8) (layer "F.Cu") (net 23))
 (via (at 126.75 111.75) (size 2) (drill 0.8) (layers "F.Cu" "B.Cu") (free) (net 23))
 (via (at 119.75 99.75) (size 2) (drill 0.8) (layers "F.Cu" "B.Cu") (free) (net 23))
 (segment (start 137.85 105.55) (end 140.05 105.55) (width 0.8) (layer "F.Cu") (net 25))
 (segment (start 140.5 106) (end 140.5 114.25) (width 0.8) (layer "F.Cu") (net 25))
 (segment (start 140.94 114.69) (end 143.75 114.69) (width 0.8) (layer "F.Cu") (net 25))
 (segment (start 140.05 105.55) (end 140.5 106) (width 0.8) (layer "F.Cu") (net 25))
 (segment (start 140.5 114.25) (end 140.94 114.69) (width 0.8) (layer "F.Cu") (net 25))
 (segment (start 122.6 103.5) (end 122.65 103.55) (width 0.8) (layer "F.Cu") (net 8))
 (segment (start 119.8 103.55) (end 119.75 103.5) (width 0.8) (layer "F.Cu") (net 8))
 (segment (start 142.75 82.75) (end 142.75 78.5) (width 0.8) (layer "F.Cu") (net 8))
 (segment (start 122.65 103.55) (end 119.8 103.55) (width 0.8) (layer "F.Cu") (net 8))
 (via (at 142.75 82.75) (size 2) (drill 0.8) (layers "F.Cu" "B.Cu") (free) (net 8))
 (via (at 119.75 103.5) (size 2) (drill 0.8) (layers "F.Cu" "B.Cu") (free) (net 8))
 (segment (start 163.235 83.25) (end 164.235 82.25) (width 0.8) (layer "F.Cu") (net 7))
 (segment (start 155.45 81.45) (end 157.25 83.25) (width 0.8) (layer "F.Cu") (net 7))
 (segment (start 157.25 83.25) (end 163.235 83.25) (width 0.8) (layer "F.Cu") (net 7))
 (segment (start 155.45 78.5) (end 155.45 81.45) (width 0.8) (layer "F.Cu") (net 7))
 (segment (start 152.5 81.25) (end 150.58 81.25) (width 0.8) (layer "F.Cu") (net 6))
 (segment (start 150.58 81.25) (end 147.83 78.5) (width 0.8) (layer "F.Cu") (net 6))
 (segment (start 156 84.75) (end 152.5 81.25) (width 0.8) (layer "F.Cu") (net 6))
 (segment (start 164.275 84.75) (end 166.775 82.25) (width 0.8) (layer "F.Cu") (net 6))
 (segment (start 156 84.75) (end 164.275 84.75) (width 0.8) (layer "F.Cu") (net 6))
 (segment (start 119.75 107.5) (end 119.75 106.25) (width 0.8) (layer "F.Cu") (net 14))
 (segment (start 120.45 105.55) (end 122.65 105.55) (width 0.8) (layer "F.Cu") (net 14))
 (segment (start 122.6 105.5) (end 122.65 105.55) (width 0.8) (layer "F.Cu") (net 14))
 (segment (start 157.99 68.26) (end 158 68.25) (width 0.8) (layer "F.Cu") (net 14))
 (segment (start 157.99 70.88) (end 157.99 68.26) (width 0.8) (layer "F.Cu") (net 14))
 (segment (start 119.75 106.25) (end 120.45 105.55) (width 0.8) (layer "F.Cu") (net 14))
 (via (at 158 68.25) (size 2) (drill 0.8) (layers "F.Cu" "B.Cu") (free) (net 14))
 (via (at 119.75 107.5) (size 2) (drill 0.8) (layers "F.Cu" "B.Cu") (free) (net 14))
 (segment (start 171.38 82.25) (end 171.5 82.25) (width 0.8) (layer "F.Cu") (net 1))
 (segment (start 166.5 90.19) (end 171.5 85.19) (width 0.8) (layer "F.Cu") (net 1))
 (segment (start 171.5 85.19) (end 171.5 82.25) (width 0.8) (layer "F.Cu") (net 1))
 (segment (start 142.5 110.5) (end 142.5 104.5) (width 0.8) (layer "F.Cu") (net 12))
 (segment (start 160.5 101.25) (end 157.5 104.25) (width 0.8) (layer "F.Cu") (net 12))
 (segment (start 157.5 104.25) (end 157.5 112) (width 0.8) (layer "F.Cu") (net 12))
 (segment (start 158 78.51) (end 157.99 78.5) (width 0.8) (layer "F.Cu") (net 12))
 (segment (start 158 81.5) (end 158 78.51) (width 0.8) (layer "F.Cu") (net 12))
 (segment (start 153 116.5) (end 148.5 116.5) (width 0.8) (layer "F.Cu") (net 12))
 (segment (start 157.5 112) (end 153 116.5) (width 0.8) (layer "F.Cu") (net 12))
 (segment (start 158 87.5) (end 158 90.5) (width 0.8) (layer "F.Cu") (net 12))
 (segment (start 148.5 116.5) (end 142.5 110.5) (width 0.8) (layer "F.Cu") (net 12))
 (segment (start 137.85 99.55) (end 138.6 99.55) (width 0.8) (layer "F.Cu") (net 12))
 (segment (start 140.2 99.55) (end 137.85 99.55) (width 0.8) (layer "F.Cu") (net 12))
 (segment (start 142.5 104.5) (end 140.75 102.75) (width 0.8) (layer "F.Cu") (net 12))
 (segment (start 160.5 93) (end 160.5 101.25) (width 0.8) (layer "F.Cu") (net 12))
 (segment (start 140.75 100.1) (end 140.2 99.55) (width 0.8) (layer "F.Cu") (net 12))
 (segment (start 158 90.5) (end 160.5 93) (width 0.8) (layer "F.Cu") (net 12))
 (segment (start 140.75 102.75) (end 140.75 100.1) (width 0.8) (layer "F.Cu") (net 12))
 (via (at 158 81.5) (size 2) (drill 0.8) (layers "F.Cu" "B.Cu") (free) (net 12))
 (via (at 158 87.5) (size 2) (drill 0.8) (layers "F.Cu" "B.Cu") (free) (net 12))
 (segment (start 141.25 92.75) (end 145.29 88.71) (width 0.8) (layer "F.Cu") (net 9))
 (segment (start 141.25 96) (end 141.25 92.75) (width 0.8) (layer "F.Cu") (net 9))
 (segment (start 145.29 88.71) (end 145.29 78.5) (width 0.8) (layer "F.Cu") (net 9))
 (segment (start 137.85 97.55) (end 139.7 97.55) (width 0.8) (layer "F.Cu") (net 9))
 (segment (start 139.7 97.55) (end 141.25 96) (width 0.8) (layer "F.Cu") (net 9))
 (segment (start 158.75 75.5) (end 167.75 75.5) (width 0.8) (layer "F.Cu") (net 2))
 (segment (start 155.45 72.2) (end 158.75 75.5) (width 0.8) (layer "F.Cu") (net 2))
 (segment (start 155.45 70.88) (end 155.45 72.2) (width 0.8) (layer "F.Cu") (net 2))
 (segment (start 174.04 81.79) (end 174.04 82.25) (width 0.8) (layer "F.Cu") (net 2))
 (segment (start 167.75 75.5) (end 174.04 81.79) (width 0.8) (layer "F.Cu") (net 2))
 (segment (start 119.75 89.5) (end 120.75 90.5) (width 0.8) (layer "F.Cu") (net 26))
 (segment (start 124.5 90.5) (end 131.75 97.75) (width 0.8) (layer "F.Cu") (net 26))
 (segment (start 119.75 85.94) (end 119.75 89.5) (width 0.8) (layer "F.Cu") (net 26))
 (segment (start 120.75 90.5) (end 124.5 90.5) (width 0.8) (layer "F.Cu") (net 26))
 (segment (start 132.55 103.55) (end 137.85 103.55) (width 0.8) (layer "F.Cu") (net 26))
 (segment (start 131.75 97.75) (end 131.75 102.75) (width 0.8) (layer "F.Cu") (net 26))
 (segment (start 131.75 102.75) (end 132.55 103.55) (width 0.8) (layer "F.Cu") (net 26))
 (segment (start 120.25 95.5) (end 120.3 95.55) (width 0.8) (layer "F.Cu") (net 24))
 (segment (start 126.75 117.5) (end 129.44 117.5) (width 0.8) (layer "F.Cu") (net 24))
 (segment (start 129.44 117.5) (end 133.44 121.5) (width 0.8) (layer "F.Cu") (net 24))
 (segment (start 119.75 96) (end 120.25 95.5) (width 0.8) (layer "F.Cu") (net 24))
 (segment (start 120.3 95.55) (end 122.65 95.55) (width 0.8) (layer "F.Cu") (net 24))
 (segment (start 133.44 121.5) (end 137.06 121.5) (width 0.8) (layer "F.Cu") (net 24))
 (via (at 119.75 96) (size 2) (drill 0.8) (layers "F.Cu" "B.Cu") (free) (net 24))
 (via (at 126.75 117.5) (size 2) (drill 0.8) (layers "F.Cu" "B.Cu") (free) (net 24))
 (segment (start 158.44 124.06) (end 158.5 124) (width 0.8) (layer "F.Cu") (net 18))
 (segment (start 155.31 119) (end 155.31 120.81) (width 0.8) (layer "F.Cu") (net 18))
 (segment (start 131.25 109.05) (end 131.25 111.25) (width 0.8) (layer "F.Cu") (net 18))
 (segment (start 140.25 124.5) (end 151.62 124.5) (width 0.8) (layer "F.Cu") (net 18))
 (segment (start 131.25 111.25) (end 134 114) (width 0.8) (layer "F.Cu") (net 18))
 (segment (start 134.25 119.5) (end 138.5 119.5) (width 0.8) (layer "F.Cu") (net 18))
 (segment (start 151.62 124.5) (end 155.31 120.81) (width 0.8) (layer "F.Cu") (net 18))
 (segment (start 138.5 119.5) (end 139.75 120.75) (width 0.8) (layer "F.Cu") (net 18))
 (segment (start 158.5 124) (end 165 124) (width 0.8) (layer "F.Cu") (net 18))
 (segment (start 139.75 124) (end 140.25 124.5) (width 0.8) (layer "F.Cu") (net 18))
 (segment (start 134 114) (end 134 119.25) (width 0.8) (layer "F.Cu") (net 18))
 (segment (start 155.31 120.81) (end 158.5 124) (width 0.8) (layer "F.Cu") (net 18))
 (segment (start 134 119.25) (end 134.25 119.5) (width 0.8) (layer "F.Cu") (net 18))
 (segment (start 139.75 120.75) (end 139.75 124) (width 0.8) (layer "F.Cu") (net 18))
 (segment (start 121.94 83.5) (end 124.25 83.5) (width 0.8) (layer "F.Cu") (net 22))
 (segment (start 134.8 101.55) (end 137.85 101.55) (width 0.8) (layer "F.Cu") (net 22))
 (segment (start 133.5 92.75) (end 133.5 100.25) (width 0.8) (layer "F.Cu") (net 22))
 (segment (start 124.25 83.5) (end 133.5 92.75) (width 0.8) (layer "F.Cu") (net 22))
 (segment (start 133.5 100.25) (end 134.8 101.55) (width 0.8) (layer "F.Cu") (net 22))
 (segment (start 122.64 93.56) (end 122.65 93.55) (width 0.8) (layer "F.Cu") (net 27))
 (segment (start 137.85 93.55) (end 137.85 89.9) (width 0.8) (layer "F.Cu") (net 20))
 (segment (start 137.85 89.9) (end 140.5 87.25) (width 0.8) (layer "F.Cu") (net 20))
 (segment (start 140.5 87.25) (end 140.5 81.88) (width 0.8) (layer "F.Cu") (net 20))
 (segment (start 140.5 81.88) (end 138.62 80) (width 0.8) (layer "F.Cu") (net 20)))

